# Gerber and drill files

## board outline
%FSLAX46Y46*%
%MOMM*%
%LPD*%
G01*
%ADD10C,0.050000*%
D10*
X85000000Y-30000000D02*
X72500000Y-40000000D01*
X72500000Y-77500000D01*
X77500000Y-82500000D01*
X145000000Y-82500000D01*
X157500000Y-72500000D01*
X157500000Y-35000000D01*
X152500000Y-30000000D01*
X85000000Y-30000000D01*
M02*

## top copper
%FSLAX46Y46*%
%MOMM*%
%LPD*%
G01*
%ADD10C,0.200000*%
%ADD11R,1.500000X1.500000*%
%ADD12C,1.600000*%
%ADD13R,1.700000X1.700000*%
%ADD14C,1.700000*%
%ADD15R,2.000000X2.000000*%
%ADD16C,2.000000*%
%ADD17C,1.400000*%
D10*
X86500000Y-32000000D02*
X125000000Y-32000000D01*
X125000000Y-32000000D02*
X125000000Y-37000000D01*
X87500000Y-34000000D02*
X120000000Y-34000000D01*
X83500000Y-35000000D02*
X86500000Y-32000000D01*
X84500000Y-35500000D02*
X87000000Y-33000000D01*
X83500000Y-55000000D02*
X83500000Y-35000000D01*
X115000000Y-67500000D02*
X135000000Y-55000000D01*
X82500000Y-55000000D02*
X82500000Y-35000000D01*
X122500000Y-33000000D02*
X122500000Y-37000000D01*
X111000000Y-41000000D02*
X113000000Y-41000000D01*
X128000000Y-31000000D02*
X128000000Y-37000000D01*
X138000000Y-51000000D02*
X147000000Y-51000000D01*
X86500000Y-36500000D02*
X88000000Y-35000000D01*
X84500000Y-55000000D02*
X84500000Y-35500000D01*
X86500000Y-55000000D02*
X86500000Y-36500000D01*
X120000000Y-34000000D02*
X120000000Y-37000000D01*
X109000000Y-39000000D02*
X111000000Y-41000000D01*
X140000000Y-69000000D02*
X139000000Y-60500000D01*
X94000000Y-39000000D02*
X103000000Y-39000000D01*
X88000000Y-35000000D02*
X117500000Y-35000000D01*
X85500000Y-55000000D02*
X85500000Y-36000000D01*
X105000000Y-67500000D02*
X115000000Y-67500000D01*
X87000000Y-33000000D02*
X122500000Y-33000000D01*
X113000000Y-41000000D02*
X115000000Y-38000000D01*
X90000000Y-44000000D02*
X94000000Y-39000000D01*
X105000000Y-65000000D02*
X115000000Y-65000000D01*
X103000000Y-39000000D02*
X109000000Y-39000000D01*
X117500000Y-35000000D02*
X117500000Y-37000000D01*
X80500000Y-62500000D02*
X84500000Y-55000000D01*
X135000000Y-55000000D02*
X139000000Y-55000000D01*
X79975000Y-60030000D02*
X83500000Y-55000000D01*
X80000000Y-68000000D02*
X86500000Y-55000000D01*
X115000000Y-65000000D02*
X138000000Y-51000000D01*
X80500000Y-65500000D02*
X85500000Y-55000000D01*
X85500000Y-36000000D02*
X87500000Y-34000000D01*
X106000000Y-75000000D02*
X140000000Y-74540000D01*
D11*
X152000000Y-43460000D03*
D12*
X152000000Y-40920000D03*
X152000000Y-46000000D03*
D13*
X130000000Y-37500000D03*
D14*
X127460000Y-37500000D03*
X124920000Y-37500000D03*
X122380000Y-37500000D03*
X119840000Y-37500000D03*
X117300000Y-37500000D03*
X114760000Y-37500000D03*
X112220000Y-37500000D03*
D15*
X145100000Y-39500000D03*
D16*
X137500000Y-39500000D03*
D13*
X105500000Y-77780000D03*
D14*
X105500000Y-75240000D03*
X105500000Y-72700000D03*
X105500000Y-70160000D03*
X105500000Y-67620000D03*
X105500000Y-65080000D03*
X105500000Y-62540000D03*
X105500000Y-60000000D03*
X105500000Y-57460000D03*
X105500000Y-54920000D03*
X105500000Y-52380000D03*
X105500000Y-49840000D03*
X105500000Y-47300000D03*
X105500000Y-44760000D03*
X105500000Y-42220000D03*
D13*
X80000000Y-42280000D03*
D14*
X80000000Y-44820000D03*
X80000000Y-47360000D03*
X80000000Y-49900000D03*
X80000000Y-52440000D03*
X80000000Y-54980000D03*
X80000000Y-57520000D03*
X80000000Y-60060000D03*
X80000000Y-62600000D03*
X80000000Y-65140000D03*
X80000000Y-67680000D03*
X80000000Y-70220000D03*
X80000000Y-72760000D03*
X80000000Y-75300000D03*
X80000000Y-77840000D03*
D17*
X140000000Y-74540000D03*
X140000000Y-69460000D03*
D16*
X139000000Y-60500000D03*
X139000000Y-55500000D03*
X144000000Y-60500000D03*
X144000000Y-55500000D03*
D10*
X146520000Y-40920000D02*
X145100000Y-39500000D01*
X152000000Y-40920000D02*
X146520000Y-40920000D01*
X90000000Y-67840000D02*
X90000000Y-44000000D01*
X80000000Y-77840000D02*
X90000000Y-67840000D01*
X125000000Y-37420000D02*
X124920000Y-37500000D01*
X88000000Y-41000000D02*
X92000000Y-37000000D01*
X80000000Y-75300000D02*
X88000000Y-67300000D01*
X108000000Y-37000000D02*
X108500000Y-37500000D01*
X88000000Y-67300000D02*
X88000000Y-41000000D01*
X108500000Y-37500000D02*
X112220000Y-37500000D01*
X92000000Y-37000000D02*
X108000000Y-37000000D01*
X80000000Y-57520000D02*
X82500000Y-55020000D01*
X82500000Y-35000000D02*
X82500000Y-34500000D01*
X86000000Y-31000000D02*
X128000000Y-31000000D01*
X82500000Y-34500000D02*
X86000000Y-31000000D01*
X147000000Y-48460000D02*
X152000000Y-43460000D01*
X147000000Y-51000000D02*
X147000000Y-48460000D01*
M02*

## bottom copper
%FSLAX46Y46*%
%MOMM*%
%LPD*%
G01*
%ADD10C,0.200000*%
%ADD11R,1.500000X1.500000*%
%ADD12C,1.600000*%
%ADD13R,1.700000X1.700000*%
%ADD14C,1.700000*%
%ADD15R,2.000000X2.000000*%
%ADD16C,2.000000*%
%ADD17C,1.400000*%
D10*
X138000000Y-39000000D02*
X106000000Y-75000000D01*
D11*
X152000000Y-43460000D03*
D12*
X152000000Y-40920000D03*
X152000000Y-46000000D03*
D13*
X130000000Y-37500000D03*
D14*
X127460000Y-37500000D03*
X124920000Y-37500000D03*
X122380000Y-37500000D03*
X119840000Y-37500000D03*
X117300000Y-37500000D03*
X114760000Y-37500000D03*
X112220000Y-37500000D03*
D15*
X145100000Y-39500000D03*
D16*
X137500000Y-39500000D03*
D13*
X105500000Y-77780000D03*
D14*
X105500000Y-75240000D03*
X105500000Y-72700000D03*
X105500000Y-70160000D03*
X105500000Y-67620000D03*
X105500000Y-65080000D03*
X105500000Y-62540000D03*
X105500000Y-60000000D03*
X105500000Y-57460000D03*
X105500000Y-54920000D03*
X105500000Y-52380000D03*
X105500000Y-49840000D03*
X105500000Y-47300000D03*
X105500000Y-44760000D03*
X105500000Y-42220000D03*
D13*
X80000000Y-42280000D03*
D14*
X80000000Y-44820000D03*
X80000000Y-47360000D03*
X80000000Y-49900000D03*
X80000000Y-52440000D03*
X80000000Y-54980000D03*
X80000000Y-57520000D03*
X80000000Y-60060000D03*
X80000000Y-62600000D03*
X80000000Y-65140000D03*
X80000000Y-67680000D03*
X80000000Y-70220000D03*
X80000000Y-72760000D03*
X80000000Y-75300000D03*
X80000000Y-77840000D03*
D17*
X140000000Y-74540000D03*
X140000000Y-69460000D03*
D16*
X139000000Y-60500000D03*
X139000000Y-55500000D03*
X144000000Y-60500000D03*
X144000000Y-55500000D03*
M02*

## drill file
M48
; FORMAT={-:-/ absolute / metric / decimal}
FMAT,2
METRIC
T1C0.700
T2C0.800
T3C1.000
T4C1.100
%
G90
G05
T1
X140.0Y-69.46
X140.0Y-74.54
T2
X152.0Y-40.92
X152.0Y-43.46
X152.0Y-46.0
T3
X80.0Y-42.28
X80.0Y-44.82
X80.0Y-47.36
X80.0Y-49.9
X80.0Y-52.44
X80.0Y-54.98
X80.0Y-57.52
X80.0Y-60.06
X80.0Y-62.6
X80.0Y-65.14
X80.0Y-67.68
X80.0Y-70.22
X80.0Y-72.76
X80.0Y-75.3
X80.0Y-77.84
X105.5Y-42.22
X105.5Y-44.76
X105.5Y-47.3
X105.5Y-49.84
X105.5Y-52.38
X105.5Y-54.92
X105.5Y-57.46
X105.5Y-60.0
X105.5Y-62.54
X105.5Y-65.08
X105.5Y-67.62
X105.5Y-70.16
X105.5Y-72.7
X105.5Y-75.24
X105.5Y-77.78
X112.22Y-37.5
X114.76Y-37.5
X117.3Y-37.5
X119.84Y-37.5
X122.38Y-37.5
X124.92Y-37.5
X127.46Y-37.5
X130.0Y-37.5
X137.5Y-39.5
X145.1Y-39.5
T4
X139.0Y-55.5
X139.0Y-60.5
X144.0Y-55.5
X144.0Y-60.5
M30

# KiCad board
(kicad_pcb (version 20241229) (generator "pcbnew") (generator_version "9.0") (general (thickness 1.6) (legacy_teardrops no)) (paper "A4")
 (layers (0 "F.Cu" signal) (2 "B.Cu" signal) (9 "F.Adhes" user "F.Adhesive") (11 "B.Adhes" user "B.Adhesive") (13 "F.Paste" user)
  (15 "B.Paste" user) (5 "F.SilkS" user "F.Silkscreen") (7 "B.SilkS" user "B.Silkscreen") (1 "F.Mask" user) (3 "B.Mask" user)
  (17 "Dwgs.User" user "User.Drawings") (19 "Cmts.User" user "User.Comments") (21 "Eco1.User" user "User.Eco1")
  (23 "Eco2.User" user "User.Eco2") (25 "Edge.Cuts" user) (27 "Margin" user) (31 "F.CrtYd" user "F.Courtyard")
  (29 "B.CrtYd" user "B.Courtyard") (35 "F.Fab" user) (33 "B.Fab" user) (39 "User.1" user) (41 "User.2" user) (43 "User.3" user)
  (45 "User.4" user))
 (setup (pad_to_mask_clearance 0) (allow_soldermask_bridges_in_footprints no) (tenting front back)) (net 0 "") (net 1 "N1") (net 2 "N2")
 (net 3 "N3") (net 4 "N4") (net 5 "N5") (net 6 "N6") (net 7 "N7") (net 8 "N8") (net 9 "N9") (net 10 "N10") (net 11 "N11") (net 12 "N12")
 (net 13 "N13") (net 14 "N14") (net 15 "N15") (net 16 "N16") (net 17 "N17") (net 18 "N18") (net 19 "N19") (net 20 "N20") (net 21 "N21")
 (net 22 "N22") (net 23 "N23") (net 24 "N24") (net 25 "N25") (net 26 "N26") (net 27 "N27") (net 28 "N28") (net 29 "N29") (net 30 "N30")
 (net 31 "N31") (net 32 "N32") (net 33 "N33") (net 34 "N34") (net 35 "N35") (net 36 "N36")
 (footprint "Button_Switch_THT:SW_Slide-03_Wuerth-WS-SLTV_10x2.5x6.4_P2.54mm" (layer "F.Cu") (at 152 43.46 -90)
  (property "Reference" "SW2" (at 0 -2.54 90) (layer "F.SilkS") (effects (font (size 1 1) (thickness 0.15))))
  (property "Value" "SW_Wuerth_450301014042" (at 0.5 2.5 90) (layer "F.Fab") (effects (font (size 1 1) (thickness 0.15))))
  (pad "1" thru_hole rect (at 0 0 270) (size 1.5 1.5) (drill 0.8) (layers "*.Cu" "*.Mask") (remove_unused_layers no) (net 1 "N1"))
  (pad "2" thru_hole circle (at -2.54 0 270) (size 1.6 1.6) (drill 0.8) (layers "*.Cu" "*.Mask") (remove_unused_layers no) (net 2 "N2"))
  (pad "3" thru_hole circle (at 2.54 0 270) (size 1.6 1.6) (drill 0.8) (layers "*.Cu" "*.Mask") (remove_unused_layers no) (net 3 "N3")))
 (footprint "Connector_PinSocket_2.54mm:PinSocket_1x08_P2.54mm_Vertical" (layer "F.Cu") (at 130 37.5 -90)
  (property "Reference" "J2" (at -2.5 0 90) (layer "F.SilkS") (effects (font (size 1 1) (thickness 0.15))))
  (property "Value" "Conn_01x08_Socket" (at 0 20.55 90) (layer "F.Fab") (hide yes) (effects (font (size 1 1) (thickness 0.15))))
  (pad "1" thru_hole rect (at 0 0 270) (size 1.7 1.7) (drill 1) (layers "*.Cu" "*.Mask") (remove_unused_layers no) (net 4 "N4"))
  (pad "2" thru_hole circle (at 0 2.54 270) (size 1.7 1.7) (drill 1) (layers "*.Cu" "*.Mask") (remove_unused_layers no) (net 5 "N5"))
  (pad "3" thru_hole circle (at 0 5.08 270) (size 1.7 1.7) (drill 1) (layers "*.Cu" "*.Mask") (remove_unused_layers no) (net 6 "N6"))
  (pad "4" thru_hole circle (at 0 7.62 270) (size 1.7 1.7) (drill 1) (layers "*.Cu" "*.Mask") (remove_unused_layers no) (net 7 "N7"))
  (pad "5" thru_hole circle (at 0 10.16 270) (size 1.7 1.7) (drill 1) (layers "*.Cu" "*.Mask") (remove_unused_layers no) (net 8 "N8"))
  (pad "6" thru_hole circle (at 0 12.7 270) (size 1.7 1.7) (drill 1) (layers "*.Cu" "*.Mask") (remove_unused_layers no) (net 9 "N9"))
  (pad "7" thru_hole circle (at 0 15.24 270) (size 1.7 1.7) (drill 1) (layers "*.Cu" "*.Mask") (remove_unused_layers no) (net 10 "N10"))
  (pad "8" thru_hole circle (at 0 17.78 270) (size 1.7 1.7) (drill 1) (layers "*.Cu" "*.Mask") (remove_unused_layers no) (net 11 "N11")))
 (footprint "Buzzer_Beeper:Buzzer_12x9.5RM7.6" (layer "F.Cu") (at 145.1 39.5 180)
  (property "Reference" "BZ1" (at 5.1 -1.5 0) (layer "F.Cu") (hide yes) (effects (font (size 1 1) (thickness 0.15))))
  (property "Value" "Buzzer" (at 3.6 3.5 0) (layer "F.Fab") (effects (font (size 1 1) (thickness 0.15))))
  (pad "1" thru_hole rect (at 0 0 180) (size 2 2) (drill 1) (layers "*.Cu" "*.Mask") (remove_unused_layers no) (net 2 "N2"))
  (pad "2" thru_hole circle (at 7.6 0 180) (size 2 2) (drill 1) (layers "*.Cu" "*.Mask") (remove_unused_layers no) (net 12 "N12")))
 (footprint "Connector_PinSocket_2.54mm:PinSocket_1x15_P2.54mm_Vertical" (layer "F.Cu") (at 105.5 77.78 180)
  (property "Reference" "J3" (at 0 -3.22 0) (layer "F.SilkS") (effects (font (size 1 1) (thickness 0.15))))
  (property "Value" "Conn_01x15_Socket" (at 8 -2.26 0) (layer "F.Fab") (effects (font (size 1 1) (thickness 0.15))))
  (pad "1" thru_hole rect (at 0 0 180) (size 1.7 1.7) (drill 1) (layers "*.Cu" "*.Mask") (remove_unused_layers no) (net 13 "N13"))
  (pad "2" thru_hole circle (at 0 2.54 180) (size 1.7 1.7) (drill 1) (layers "*.Cu" "*.Mask") (remove_unused_layers no) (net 12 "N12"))
  (pad "3" thru_hole circle (at 0 5.08 180) (size 1.7 1.7) (drill 1) (layers "*.Cu" "*.Mask") (remove_unused_layers no) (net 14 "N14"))
  (pad "4" thru_hole circle (at 0 7.62 180) (size 1.7 1.7) (drill 1) (layers "*.Cu" "*.Mask") (remove_unused_layers no) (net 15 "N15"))
  (pad "5" thru_hole circle (at 0 10.16 180) (size 1.7 1.7) (drill 1) (layers "*.Cu" "*.Mask") (remove_unused_layers no) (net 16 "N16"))
  (pad "6" thru_hole circle (at 0 12.7 180) (size 1.7 1.7) (drill 1) (layers "*.Cu" "*.Mask") (remove_unused_layers no) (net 1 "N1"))
  (pad "7" thru_hole circle (at 0 15.24 180) (size 1.7 1.7) (drill 1) (layers "*.Cu" "*.Mask") (remove_unused_layers no) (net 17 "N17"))
  (pad "8" thru_hole circle (at 0 17.78 180) (size 1.7 1.7) (drill 1) (layers "*.Cu" "*.Mask") (remove_unused_layers no) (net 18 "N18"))
  (pad "9" thru_hole circle (at 0 20.32 180) (size 1.7 1.7) (drill 1) (layers "*.Cu" "*.Mask") (remove_unused_layers no) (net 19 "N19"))
  (pad "10" thru_hole circle (at 0 22.86 180) (size 1.7 1.7) (drill 1) (layers "*.Cu" "*.Mask") (remove_unused_layers no) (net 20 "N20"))
  (pad "11" thru_hole circle (at 0 25.4 180) (size 1.7 1.7) (drill 1) (layers "*.Cu" "*.Mask") (remove_unused_layers no) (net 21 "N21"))
  (pad "12" thru_hole circle (at 0 27.94 180) (size 1.7 1.7) (drill 1) (layers "*.Cu" "*.Mask") (remove_unused_layers no) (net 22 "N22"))
  (pad "13" thru_hole circle (at 0 30.48 180) (size 1.7 1.7) (drill 1) (layers "*.Cu" "*.Mask") (remove_unused_layers no) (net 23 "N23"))
  (pad "14" thru_hole circle (at 0 33.02 180) (size 1.7 1.7) (drill 1) (layers "*.Cu" "*.Mask") (remove_unused_layers no) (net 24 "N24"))
  (pad "15" thru_hole circle (at 0 35.56 180) (size 1.7 1.7) (drill 1) (layers "*.Cu" "*.Mask") (remove_unused_layers no) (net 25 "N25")))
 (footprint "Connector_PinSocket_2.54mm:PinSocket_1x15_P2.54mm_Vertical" (layer "F.Cu") (at 80 42.28)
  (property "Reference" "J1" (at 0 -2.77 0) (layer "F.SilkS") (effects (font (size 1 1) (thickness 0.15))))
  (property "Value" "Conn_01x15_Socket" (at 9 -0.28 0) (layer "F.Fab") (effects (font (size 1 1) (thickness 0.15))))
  (pad "1" thru_hole rect (at 0 0) (size 1.7 1.7) (drill 1) (layers "*.Cu" "*.Mask") (remove_unused_layers no) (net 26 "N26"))
  (pad "2" thru_hole circle (at 0 2.54) (size 1.7 1.7) (drill 1) (layers "*.Cu" "*.Mask") (remove_unused_layers no) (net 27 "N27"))
  (pad "3" thru_hole circle (at 0 5.08) (size 1.7 1.7) (drill 1) (layers "*.Cu" "*.Mask") (remove_unused_layers no) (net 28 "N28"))
  (pad "4" thru_hole circle (at 0 7.62) (size 1.7 1.7) (drill 1) (layers "*.Cu" "*.Mask") (remove_unused_layers no) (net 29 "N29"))
  (pad "5" thru_hole circle (at 0 10.16) (size 1.7 1.7) (drill 1) (layers "*.Cu" "*.Mask") (remove_unused_layers no) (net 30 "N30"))
  (pad "6" thru_hole circle (at 0 12.7) (size 1.7 1.7) (drill 1) (layers "*.Cu" "*.Mask") (remove_unused_layers no) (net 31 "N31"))
  (pad "7" thru_hole circle (at 0 15.24) (size 1.7 1.7) (drill 1) (layers "*.Cu" "*.Mask") (remove_unused_layers no) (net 5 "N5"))
  (pad "8" thru_hole circle (at 0 17.78) (size 1.7 1.7) (drill 1) (layers "*.Cu" "*.Mask") (remove_unused_layers no) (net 6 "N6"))
  (pad "9" thru_hole circle (at 0 20.32) (size 1.7 1.7) (drill 1) (layers "*.Cu" "*.Mask") (remove_unused_layers no) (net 7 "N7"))
  (pad "10" thru_hole circle (at 0 22.86) (size 1.7 1.7) (drill 1) (layers "*.Cu" "*.Mask") (remove_unused_layers no) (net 8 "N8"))
  (pad "11" thru_hole circle (at 0 25.4) (size 1.7 1.7) (drill 1) (layers "*.Cu" "*.Mask") (remove_unused_layers no) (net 9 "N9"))
  (pad "12" thru_hole circle (at 0 27.94) (size 1.7 1.7) (drill 1) (layers "*.Cu" "*.Mask") (remove_unused_layers no) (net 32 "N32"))
  (pad "13" thru_hole circle (at 0 30.48) (size 1.7 1.7) (drill 1) (layers "*.Cu" "*.Mask") (remove_unused_layers no) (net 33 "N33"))
  (pad "14" thru_hole circle (at 0 33.02) (size 1.7 1.7) (drill 1) (layers "*.Cu" "*.Mask") (remove_unused_layers no) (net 11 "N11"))
  (pad "15" thru_hole circle (at 0 35.56) (size 1.7 1.7) (drill 1) (layers "*.Cu" "*.Mask") (remove_unused_layers no) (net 10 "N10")))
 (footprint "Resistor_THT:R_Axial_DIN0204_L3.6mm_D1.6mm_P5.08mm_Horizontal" (layer "F.Cu") (at 140 74.54 90)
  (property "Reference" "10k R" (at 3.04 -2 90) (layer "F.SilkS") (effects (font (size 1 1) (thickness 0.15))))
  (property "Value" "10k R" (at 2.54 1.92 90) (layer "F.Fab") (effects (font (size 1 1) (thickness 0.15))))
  (pad "1" thru_hole circle (at 0 0 90) (size 1.4 1.4) (drill 0.7) (layers "*.Cu" "*.Mask") (remove_unused_layers no) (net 12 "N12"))
  (pad "2" thru_hole circle (at 5.08 0 90) (size 1.4 1.4) (drill 0.7) (layers "*.Cu" "*.Mask") (remove_unused_layers no) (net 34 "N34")))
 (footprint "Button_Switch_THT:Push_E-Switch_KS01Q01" (layer "F.Cu") (at 139 60.5 90)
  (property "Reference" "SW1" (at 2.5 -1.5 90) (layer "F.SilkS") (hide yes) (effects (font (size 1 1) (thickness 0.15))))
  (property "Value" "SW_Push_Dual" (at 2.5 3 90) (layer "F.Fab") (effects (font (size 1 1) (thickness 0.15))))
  (pad "1" thru_hole circle (at 0 0 90) (size 2 2) (drill 1.1) (layers "*.Cu" "*.Mask") (remove_unused_layers no) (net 34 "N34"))
  (pad "2" thru_hole circle (at 5 0 90) (size 2 2) (drill 1.1) (layers "*.Cu" "*.Mask") (remove_unused_layers no) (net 16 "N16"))
  (pad "3" thru_hole circle (at 0 5 90) (size 2 2) (drill 1.1) (layers "*.Cu" "*.Mask") (remove_unused_layers no) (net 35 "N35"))
  (pad "4" thru_hole circle (at 5 5 90) (size 2 2) (drill 1.1) (layers "*.Cu" "*.Mask") (remove_unused_layers no) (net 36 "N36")))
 (gr_line (start 86.5 32) (end 125 32) (stroke (width 0.2) (type default)) (layer "F.Cu") (net 6))
 (gr_line (start 125 32) (end 125 37) (stroke (width 0.2) (type default)) (layer "F.Cu") (net 6))
 (gr_line (start 87.5 34) (end 120 34) (stroke (width 0.2) (type default)) (layer "F.Cu") (net 8))
 (gr_line (start 83.5 35) (end 86.5 32) (stroke (width 0.2) (type default)) (layer "F.Cu") (net 6))
 (gr_line (start 84.5 35.5) (end 87 33) (stroke (width 0.2) (type default)) (layer "F.Cu") (net 7))
 (gr_line (start 83.5 55) (end 83.5 35) (stroke (width 0.2) (type default)) (layer "F.Cu") (net 6))
 (gr_line (start 115 67.5) (end 135 55) (stroke (width 0.2) (type default)) (layer "F.Cu") (net 16))
 (gr_line (start 82.5 55) (end 82.5 35) (stroke (width 0.2) (type default)) (layer "F.Cu") (net 5))
 (gr_line (start 122.5 33) (end 122.5 37) (stroke (width 0.2) (type default)) (layer "F.Cu") (net 7))
 (gr_line (start 111 41) (end 113 41) (stroke (width 0.2) (type default)) (layer "F.Cu") (net 10))
 (gr_line (start 128 31) (end 128 37) (stroke (width 0.2) (type default)) (layer "F.Cu") (net 5))
 (gr_line (start 138 51) (end 147 51) (stroke (width 0.2) (type default)) (layer "F.Cu") (net 1))
 (gr_line (start 86.5 36.5) (end 88 35) (stroke (width 0.2) (type default)) (layer "F.Cu") (net 9))
 (gr_line (start 84.5 55) (end 84.5 35.5) (stroke (width 0.2) (type default)) (layer "F.Cu") (net 7))
 (gr_line (start 86.5 55) (end 86.5 36.5) (stroke (width 0.2) (type default)) (layer "F.Cu") (net 9))
 (gr_line (start 120 34) (end 120 37) (stroke (width 0.2) (type default)) (layer "F.Cu") (net 8))
 (gr_line (start 109 39) (end 111 41) (stroke (width 0.2) (type default)) (layer "F.Cu") (net 10))
 (gr_line (start 140 69) (end 139 60.5) (stroke (width 0.2) (type default)) (layer "F.Cu") (net 34))
 (gr_line (start 94 39) (end 103 39) (stroke (width 0.2) (type default)) (layer "F.Cu") (net 10))
 (gr_line (start 88 35) (end 117.5 35) (stroke (width 0.2) (type default)) (layer "F.Cu") (net 9))
 (gr_line (start 85.5 55) (end 85.5 36) (stroke (width 0.2) (type default)) (layer "F.Cu") (net 8))
 (gr_line (start 105 67.5) (end 115 67.5) (stroke (width 0.2) (type default)) (layer "F.Cu") (net 16))
 (gr_line (start 87 33) (end 122.5 33) (stroke (width 0.2) (type default)) (layer "F.Cu") (net 7))
 (gr_line (start 113 41) (end 115 38) (stroke (width 0.2) (type default)) (layer "F.Cu") (net 10))
 (gr_line (start 90 44) (end 94 39) (stroke (width 0.2) (type default)) (layer "F.Cu") (net 10))
 (gr_line (start 105 65) (end 115 65) (stroke (width 0.2) (type default)) (layer "F.Cu") (net 1))
 (gr_line (start 103 39) (end 109 39) (stroke (width 0.2) (type default)) (layer "F.Cu") (net 10))
 (gr_line (start 117.5 35) (end 117.5 37) (stroke (width 0.2) (type default)) (layer "F.Cu") (net 9))
 (gr_line (start 80.5 62.5) (end 84.5 55) (stroke (width 0.2) (type default)) (layer "F.Cu") (net 7))
 (gr_line (start 135 55) (end 139 55) (stroke (width 0.2) (type default)) (layer "F.Cu") (net 16))
 (gr_line (start 79.975 60.03) (end 83.5 55) (stroke (width 0.2) (type default)) (layer "F.Cu") (net 6))
 (gr_line (start 80 68) (end 86.5 55) (stroke (width 0.2) (type default)) (layer "F.Cu") (net 9))
 (gr_line (start 115 65) (end 138 51) (stroke (width 0.2) (type default)) (layer "F.Cu") (net 1))
 (gr_line (start 80.5 65.5) (end 85.5 55) (stroke (width 0.2) (type default)) (layer "F.Cu") (net 8))
 (gr_line (start 85.5 36) (end 87.5 34) (stroke (width 0.2) (type default)) (layer "F.Cu") (net 8))
 (gr_line (start 106 75) (end 140 74.54) (stroke (width 0.2) (type default)) (layer "F.Cu") (net 12))
 (gr_line (start 138 39) (end 106 75) (stroke (width 0.2) (type default)) (layer "B.Cu") (net 12))
 (gr_poly
  (pts (xy 85 30) (xy 72.5 40) (xy 72.5 77.5) (xy 77.5 82.5) (xy 145 82.5) (xy 157.5 72.5) (xy 157.5 35) (xy 152.5 30))
  (stroke (width 0.05) (type solid)) (fill no) (layer "Edge.Cuts"))
 (segment (start 146.52 40.92) (end 145.1 39.5) (width 0.2) (layer "F.Cu") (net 2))
 (segment (start 152 40.92) (end 146.52 40.92) (width 0.2) (layer "F.Cu") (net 2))
 (segment (start 90 67.84) (end 90 44) (width 0.2) (layer "F.Cu") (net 10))
 (segment (start 80 77.84) (end 90 67.84) (width 0.2) (layer "F.Cu") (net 10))
 (segment (start 125 37.42) (end 124.92 37.5) (width 0.2) (layer "F.Cu") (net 6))
 (segment (start 88 41) (end 92 37) (width 0.2) (layer "F.Cu") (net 11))
 (segment (start 80 75.3) (end 88 67.3) (width 0.2) (layer "F.Cu") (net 11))
 (segment (start 108 37) (end 108.5 37.5) (width 0.2) (layer "F.Cu") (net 11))
 (segment (start 88 67.3) (end 88 41) (width 0.2) (layer "F.Cu") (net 11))
 (segment (start 108.5 37.5) (end 112.22 37.5) (width 0.2) (layer "F.Cu") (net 11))
 (segment (start 92 37) (end 108 37) (width 0.2) (layer "F.Cu") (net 11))
 (segment (start 80 57.52) (end 82.5 55.02) (width 0.2) (layer "F.Cu") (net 5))
 (segment (start 82.5 35) (end 82.5 34.5) (width 0.2) (layer "F.Cu") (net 5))
 (segment (start 86 31) (end 128 31) (width 0.2) (layer "F.Cu") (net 5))
 (segment (start 82.5 34.5) (end 86 31) (width 0.2) (layer "F.Cu") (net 5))
 (segment (start 147 48.46) (end 152 43.46) (width 0.2) (layer "F.Cu") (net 1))
 (segment (start 147 51) (end 147 48.46) (width 0.2) (layer "F.Cu") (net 1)))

